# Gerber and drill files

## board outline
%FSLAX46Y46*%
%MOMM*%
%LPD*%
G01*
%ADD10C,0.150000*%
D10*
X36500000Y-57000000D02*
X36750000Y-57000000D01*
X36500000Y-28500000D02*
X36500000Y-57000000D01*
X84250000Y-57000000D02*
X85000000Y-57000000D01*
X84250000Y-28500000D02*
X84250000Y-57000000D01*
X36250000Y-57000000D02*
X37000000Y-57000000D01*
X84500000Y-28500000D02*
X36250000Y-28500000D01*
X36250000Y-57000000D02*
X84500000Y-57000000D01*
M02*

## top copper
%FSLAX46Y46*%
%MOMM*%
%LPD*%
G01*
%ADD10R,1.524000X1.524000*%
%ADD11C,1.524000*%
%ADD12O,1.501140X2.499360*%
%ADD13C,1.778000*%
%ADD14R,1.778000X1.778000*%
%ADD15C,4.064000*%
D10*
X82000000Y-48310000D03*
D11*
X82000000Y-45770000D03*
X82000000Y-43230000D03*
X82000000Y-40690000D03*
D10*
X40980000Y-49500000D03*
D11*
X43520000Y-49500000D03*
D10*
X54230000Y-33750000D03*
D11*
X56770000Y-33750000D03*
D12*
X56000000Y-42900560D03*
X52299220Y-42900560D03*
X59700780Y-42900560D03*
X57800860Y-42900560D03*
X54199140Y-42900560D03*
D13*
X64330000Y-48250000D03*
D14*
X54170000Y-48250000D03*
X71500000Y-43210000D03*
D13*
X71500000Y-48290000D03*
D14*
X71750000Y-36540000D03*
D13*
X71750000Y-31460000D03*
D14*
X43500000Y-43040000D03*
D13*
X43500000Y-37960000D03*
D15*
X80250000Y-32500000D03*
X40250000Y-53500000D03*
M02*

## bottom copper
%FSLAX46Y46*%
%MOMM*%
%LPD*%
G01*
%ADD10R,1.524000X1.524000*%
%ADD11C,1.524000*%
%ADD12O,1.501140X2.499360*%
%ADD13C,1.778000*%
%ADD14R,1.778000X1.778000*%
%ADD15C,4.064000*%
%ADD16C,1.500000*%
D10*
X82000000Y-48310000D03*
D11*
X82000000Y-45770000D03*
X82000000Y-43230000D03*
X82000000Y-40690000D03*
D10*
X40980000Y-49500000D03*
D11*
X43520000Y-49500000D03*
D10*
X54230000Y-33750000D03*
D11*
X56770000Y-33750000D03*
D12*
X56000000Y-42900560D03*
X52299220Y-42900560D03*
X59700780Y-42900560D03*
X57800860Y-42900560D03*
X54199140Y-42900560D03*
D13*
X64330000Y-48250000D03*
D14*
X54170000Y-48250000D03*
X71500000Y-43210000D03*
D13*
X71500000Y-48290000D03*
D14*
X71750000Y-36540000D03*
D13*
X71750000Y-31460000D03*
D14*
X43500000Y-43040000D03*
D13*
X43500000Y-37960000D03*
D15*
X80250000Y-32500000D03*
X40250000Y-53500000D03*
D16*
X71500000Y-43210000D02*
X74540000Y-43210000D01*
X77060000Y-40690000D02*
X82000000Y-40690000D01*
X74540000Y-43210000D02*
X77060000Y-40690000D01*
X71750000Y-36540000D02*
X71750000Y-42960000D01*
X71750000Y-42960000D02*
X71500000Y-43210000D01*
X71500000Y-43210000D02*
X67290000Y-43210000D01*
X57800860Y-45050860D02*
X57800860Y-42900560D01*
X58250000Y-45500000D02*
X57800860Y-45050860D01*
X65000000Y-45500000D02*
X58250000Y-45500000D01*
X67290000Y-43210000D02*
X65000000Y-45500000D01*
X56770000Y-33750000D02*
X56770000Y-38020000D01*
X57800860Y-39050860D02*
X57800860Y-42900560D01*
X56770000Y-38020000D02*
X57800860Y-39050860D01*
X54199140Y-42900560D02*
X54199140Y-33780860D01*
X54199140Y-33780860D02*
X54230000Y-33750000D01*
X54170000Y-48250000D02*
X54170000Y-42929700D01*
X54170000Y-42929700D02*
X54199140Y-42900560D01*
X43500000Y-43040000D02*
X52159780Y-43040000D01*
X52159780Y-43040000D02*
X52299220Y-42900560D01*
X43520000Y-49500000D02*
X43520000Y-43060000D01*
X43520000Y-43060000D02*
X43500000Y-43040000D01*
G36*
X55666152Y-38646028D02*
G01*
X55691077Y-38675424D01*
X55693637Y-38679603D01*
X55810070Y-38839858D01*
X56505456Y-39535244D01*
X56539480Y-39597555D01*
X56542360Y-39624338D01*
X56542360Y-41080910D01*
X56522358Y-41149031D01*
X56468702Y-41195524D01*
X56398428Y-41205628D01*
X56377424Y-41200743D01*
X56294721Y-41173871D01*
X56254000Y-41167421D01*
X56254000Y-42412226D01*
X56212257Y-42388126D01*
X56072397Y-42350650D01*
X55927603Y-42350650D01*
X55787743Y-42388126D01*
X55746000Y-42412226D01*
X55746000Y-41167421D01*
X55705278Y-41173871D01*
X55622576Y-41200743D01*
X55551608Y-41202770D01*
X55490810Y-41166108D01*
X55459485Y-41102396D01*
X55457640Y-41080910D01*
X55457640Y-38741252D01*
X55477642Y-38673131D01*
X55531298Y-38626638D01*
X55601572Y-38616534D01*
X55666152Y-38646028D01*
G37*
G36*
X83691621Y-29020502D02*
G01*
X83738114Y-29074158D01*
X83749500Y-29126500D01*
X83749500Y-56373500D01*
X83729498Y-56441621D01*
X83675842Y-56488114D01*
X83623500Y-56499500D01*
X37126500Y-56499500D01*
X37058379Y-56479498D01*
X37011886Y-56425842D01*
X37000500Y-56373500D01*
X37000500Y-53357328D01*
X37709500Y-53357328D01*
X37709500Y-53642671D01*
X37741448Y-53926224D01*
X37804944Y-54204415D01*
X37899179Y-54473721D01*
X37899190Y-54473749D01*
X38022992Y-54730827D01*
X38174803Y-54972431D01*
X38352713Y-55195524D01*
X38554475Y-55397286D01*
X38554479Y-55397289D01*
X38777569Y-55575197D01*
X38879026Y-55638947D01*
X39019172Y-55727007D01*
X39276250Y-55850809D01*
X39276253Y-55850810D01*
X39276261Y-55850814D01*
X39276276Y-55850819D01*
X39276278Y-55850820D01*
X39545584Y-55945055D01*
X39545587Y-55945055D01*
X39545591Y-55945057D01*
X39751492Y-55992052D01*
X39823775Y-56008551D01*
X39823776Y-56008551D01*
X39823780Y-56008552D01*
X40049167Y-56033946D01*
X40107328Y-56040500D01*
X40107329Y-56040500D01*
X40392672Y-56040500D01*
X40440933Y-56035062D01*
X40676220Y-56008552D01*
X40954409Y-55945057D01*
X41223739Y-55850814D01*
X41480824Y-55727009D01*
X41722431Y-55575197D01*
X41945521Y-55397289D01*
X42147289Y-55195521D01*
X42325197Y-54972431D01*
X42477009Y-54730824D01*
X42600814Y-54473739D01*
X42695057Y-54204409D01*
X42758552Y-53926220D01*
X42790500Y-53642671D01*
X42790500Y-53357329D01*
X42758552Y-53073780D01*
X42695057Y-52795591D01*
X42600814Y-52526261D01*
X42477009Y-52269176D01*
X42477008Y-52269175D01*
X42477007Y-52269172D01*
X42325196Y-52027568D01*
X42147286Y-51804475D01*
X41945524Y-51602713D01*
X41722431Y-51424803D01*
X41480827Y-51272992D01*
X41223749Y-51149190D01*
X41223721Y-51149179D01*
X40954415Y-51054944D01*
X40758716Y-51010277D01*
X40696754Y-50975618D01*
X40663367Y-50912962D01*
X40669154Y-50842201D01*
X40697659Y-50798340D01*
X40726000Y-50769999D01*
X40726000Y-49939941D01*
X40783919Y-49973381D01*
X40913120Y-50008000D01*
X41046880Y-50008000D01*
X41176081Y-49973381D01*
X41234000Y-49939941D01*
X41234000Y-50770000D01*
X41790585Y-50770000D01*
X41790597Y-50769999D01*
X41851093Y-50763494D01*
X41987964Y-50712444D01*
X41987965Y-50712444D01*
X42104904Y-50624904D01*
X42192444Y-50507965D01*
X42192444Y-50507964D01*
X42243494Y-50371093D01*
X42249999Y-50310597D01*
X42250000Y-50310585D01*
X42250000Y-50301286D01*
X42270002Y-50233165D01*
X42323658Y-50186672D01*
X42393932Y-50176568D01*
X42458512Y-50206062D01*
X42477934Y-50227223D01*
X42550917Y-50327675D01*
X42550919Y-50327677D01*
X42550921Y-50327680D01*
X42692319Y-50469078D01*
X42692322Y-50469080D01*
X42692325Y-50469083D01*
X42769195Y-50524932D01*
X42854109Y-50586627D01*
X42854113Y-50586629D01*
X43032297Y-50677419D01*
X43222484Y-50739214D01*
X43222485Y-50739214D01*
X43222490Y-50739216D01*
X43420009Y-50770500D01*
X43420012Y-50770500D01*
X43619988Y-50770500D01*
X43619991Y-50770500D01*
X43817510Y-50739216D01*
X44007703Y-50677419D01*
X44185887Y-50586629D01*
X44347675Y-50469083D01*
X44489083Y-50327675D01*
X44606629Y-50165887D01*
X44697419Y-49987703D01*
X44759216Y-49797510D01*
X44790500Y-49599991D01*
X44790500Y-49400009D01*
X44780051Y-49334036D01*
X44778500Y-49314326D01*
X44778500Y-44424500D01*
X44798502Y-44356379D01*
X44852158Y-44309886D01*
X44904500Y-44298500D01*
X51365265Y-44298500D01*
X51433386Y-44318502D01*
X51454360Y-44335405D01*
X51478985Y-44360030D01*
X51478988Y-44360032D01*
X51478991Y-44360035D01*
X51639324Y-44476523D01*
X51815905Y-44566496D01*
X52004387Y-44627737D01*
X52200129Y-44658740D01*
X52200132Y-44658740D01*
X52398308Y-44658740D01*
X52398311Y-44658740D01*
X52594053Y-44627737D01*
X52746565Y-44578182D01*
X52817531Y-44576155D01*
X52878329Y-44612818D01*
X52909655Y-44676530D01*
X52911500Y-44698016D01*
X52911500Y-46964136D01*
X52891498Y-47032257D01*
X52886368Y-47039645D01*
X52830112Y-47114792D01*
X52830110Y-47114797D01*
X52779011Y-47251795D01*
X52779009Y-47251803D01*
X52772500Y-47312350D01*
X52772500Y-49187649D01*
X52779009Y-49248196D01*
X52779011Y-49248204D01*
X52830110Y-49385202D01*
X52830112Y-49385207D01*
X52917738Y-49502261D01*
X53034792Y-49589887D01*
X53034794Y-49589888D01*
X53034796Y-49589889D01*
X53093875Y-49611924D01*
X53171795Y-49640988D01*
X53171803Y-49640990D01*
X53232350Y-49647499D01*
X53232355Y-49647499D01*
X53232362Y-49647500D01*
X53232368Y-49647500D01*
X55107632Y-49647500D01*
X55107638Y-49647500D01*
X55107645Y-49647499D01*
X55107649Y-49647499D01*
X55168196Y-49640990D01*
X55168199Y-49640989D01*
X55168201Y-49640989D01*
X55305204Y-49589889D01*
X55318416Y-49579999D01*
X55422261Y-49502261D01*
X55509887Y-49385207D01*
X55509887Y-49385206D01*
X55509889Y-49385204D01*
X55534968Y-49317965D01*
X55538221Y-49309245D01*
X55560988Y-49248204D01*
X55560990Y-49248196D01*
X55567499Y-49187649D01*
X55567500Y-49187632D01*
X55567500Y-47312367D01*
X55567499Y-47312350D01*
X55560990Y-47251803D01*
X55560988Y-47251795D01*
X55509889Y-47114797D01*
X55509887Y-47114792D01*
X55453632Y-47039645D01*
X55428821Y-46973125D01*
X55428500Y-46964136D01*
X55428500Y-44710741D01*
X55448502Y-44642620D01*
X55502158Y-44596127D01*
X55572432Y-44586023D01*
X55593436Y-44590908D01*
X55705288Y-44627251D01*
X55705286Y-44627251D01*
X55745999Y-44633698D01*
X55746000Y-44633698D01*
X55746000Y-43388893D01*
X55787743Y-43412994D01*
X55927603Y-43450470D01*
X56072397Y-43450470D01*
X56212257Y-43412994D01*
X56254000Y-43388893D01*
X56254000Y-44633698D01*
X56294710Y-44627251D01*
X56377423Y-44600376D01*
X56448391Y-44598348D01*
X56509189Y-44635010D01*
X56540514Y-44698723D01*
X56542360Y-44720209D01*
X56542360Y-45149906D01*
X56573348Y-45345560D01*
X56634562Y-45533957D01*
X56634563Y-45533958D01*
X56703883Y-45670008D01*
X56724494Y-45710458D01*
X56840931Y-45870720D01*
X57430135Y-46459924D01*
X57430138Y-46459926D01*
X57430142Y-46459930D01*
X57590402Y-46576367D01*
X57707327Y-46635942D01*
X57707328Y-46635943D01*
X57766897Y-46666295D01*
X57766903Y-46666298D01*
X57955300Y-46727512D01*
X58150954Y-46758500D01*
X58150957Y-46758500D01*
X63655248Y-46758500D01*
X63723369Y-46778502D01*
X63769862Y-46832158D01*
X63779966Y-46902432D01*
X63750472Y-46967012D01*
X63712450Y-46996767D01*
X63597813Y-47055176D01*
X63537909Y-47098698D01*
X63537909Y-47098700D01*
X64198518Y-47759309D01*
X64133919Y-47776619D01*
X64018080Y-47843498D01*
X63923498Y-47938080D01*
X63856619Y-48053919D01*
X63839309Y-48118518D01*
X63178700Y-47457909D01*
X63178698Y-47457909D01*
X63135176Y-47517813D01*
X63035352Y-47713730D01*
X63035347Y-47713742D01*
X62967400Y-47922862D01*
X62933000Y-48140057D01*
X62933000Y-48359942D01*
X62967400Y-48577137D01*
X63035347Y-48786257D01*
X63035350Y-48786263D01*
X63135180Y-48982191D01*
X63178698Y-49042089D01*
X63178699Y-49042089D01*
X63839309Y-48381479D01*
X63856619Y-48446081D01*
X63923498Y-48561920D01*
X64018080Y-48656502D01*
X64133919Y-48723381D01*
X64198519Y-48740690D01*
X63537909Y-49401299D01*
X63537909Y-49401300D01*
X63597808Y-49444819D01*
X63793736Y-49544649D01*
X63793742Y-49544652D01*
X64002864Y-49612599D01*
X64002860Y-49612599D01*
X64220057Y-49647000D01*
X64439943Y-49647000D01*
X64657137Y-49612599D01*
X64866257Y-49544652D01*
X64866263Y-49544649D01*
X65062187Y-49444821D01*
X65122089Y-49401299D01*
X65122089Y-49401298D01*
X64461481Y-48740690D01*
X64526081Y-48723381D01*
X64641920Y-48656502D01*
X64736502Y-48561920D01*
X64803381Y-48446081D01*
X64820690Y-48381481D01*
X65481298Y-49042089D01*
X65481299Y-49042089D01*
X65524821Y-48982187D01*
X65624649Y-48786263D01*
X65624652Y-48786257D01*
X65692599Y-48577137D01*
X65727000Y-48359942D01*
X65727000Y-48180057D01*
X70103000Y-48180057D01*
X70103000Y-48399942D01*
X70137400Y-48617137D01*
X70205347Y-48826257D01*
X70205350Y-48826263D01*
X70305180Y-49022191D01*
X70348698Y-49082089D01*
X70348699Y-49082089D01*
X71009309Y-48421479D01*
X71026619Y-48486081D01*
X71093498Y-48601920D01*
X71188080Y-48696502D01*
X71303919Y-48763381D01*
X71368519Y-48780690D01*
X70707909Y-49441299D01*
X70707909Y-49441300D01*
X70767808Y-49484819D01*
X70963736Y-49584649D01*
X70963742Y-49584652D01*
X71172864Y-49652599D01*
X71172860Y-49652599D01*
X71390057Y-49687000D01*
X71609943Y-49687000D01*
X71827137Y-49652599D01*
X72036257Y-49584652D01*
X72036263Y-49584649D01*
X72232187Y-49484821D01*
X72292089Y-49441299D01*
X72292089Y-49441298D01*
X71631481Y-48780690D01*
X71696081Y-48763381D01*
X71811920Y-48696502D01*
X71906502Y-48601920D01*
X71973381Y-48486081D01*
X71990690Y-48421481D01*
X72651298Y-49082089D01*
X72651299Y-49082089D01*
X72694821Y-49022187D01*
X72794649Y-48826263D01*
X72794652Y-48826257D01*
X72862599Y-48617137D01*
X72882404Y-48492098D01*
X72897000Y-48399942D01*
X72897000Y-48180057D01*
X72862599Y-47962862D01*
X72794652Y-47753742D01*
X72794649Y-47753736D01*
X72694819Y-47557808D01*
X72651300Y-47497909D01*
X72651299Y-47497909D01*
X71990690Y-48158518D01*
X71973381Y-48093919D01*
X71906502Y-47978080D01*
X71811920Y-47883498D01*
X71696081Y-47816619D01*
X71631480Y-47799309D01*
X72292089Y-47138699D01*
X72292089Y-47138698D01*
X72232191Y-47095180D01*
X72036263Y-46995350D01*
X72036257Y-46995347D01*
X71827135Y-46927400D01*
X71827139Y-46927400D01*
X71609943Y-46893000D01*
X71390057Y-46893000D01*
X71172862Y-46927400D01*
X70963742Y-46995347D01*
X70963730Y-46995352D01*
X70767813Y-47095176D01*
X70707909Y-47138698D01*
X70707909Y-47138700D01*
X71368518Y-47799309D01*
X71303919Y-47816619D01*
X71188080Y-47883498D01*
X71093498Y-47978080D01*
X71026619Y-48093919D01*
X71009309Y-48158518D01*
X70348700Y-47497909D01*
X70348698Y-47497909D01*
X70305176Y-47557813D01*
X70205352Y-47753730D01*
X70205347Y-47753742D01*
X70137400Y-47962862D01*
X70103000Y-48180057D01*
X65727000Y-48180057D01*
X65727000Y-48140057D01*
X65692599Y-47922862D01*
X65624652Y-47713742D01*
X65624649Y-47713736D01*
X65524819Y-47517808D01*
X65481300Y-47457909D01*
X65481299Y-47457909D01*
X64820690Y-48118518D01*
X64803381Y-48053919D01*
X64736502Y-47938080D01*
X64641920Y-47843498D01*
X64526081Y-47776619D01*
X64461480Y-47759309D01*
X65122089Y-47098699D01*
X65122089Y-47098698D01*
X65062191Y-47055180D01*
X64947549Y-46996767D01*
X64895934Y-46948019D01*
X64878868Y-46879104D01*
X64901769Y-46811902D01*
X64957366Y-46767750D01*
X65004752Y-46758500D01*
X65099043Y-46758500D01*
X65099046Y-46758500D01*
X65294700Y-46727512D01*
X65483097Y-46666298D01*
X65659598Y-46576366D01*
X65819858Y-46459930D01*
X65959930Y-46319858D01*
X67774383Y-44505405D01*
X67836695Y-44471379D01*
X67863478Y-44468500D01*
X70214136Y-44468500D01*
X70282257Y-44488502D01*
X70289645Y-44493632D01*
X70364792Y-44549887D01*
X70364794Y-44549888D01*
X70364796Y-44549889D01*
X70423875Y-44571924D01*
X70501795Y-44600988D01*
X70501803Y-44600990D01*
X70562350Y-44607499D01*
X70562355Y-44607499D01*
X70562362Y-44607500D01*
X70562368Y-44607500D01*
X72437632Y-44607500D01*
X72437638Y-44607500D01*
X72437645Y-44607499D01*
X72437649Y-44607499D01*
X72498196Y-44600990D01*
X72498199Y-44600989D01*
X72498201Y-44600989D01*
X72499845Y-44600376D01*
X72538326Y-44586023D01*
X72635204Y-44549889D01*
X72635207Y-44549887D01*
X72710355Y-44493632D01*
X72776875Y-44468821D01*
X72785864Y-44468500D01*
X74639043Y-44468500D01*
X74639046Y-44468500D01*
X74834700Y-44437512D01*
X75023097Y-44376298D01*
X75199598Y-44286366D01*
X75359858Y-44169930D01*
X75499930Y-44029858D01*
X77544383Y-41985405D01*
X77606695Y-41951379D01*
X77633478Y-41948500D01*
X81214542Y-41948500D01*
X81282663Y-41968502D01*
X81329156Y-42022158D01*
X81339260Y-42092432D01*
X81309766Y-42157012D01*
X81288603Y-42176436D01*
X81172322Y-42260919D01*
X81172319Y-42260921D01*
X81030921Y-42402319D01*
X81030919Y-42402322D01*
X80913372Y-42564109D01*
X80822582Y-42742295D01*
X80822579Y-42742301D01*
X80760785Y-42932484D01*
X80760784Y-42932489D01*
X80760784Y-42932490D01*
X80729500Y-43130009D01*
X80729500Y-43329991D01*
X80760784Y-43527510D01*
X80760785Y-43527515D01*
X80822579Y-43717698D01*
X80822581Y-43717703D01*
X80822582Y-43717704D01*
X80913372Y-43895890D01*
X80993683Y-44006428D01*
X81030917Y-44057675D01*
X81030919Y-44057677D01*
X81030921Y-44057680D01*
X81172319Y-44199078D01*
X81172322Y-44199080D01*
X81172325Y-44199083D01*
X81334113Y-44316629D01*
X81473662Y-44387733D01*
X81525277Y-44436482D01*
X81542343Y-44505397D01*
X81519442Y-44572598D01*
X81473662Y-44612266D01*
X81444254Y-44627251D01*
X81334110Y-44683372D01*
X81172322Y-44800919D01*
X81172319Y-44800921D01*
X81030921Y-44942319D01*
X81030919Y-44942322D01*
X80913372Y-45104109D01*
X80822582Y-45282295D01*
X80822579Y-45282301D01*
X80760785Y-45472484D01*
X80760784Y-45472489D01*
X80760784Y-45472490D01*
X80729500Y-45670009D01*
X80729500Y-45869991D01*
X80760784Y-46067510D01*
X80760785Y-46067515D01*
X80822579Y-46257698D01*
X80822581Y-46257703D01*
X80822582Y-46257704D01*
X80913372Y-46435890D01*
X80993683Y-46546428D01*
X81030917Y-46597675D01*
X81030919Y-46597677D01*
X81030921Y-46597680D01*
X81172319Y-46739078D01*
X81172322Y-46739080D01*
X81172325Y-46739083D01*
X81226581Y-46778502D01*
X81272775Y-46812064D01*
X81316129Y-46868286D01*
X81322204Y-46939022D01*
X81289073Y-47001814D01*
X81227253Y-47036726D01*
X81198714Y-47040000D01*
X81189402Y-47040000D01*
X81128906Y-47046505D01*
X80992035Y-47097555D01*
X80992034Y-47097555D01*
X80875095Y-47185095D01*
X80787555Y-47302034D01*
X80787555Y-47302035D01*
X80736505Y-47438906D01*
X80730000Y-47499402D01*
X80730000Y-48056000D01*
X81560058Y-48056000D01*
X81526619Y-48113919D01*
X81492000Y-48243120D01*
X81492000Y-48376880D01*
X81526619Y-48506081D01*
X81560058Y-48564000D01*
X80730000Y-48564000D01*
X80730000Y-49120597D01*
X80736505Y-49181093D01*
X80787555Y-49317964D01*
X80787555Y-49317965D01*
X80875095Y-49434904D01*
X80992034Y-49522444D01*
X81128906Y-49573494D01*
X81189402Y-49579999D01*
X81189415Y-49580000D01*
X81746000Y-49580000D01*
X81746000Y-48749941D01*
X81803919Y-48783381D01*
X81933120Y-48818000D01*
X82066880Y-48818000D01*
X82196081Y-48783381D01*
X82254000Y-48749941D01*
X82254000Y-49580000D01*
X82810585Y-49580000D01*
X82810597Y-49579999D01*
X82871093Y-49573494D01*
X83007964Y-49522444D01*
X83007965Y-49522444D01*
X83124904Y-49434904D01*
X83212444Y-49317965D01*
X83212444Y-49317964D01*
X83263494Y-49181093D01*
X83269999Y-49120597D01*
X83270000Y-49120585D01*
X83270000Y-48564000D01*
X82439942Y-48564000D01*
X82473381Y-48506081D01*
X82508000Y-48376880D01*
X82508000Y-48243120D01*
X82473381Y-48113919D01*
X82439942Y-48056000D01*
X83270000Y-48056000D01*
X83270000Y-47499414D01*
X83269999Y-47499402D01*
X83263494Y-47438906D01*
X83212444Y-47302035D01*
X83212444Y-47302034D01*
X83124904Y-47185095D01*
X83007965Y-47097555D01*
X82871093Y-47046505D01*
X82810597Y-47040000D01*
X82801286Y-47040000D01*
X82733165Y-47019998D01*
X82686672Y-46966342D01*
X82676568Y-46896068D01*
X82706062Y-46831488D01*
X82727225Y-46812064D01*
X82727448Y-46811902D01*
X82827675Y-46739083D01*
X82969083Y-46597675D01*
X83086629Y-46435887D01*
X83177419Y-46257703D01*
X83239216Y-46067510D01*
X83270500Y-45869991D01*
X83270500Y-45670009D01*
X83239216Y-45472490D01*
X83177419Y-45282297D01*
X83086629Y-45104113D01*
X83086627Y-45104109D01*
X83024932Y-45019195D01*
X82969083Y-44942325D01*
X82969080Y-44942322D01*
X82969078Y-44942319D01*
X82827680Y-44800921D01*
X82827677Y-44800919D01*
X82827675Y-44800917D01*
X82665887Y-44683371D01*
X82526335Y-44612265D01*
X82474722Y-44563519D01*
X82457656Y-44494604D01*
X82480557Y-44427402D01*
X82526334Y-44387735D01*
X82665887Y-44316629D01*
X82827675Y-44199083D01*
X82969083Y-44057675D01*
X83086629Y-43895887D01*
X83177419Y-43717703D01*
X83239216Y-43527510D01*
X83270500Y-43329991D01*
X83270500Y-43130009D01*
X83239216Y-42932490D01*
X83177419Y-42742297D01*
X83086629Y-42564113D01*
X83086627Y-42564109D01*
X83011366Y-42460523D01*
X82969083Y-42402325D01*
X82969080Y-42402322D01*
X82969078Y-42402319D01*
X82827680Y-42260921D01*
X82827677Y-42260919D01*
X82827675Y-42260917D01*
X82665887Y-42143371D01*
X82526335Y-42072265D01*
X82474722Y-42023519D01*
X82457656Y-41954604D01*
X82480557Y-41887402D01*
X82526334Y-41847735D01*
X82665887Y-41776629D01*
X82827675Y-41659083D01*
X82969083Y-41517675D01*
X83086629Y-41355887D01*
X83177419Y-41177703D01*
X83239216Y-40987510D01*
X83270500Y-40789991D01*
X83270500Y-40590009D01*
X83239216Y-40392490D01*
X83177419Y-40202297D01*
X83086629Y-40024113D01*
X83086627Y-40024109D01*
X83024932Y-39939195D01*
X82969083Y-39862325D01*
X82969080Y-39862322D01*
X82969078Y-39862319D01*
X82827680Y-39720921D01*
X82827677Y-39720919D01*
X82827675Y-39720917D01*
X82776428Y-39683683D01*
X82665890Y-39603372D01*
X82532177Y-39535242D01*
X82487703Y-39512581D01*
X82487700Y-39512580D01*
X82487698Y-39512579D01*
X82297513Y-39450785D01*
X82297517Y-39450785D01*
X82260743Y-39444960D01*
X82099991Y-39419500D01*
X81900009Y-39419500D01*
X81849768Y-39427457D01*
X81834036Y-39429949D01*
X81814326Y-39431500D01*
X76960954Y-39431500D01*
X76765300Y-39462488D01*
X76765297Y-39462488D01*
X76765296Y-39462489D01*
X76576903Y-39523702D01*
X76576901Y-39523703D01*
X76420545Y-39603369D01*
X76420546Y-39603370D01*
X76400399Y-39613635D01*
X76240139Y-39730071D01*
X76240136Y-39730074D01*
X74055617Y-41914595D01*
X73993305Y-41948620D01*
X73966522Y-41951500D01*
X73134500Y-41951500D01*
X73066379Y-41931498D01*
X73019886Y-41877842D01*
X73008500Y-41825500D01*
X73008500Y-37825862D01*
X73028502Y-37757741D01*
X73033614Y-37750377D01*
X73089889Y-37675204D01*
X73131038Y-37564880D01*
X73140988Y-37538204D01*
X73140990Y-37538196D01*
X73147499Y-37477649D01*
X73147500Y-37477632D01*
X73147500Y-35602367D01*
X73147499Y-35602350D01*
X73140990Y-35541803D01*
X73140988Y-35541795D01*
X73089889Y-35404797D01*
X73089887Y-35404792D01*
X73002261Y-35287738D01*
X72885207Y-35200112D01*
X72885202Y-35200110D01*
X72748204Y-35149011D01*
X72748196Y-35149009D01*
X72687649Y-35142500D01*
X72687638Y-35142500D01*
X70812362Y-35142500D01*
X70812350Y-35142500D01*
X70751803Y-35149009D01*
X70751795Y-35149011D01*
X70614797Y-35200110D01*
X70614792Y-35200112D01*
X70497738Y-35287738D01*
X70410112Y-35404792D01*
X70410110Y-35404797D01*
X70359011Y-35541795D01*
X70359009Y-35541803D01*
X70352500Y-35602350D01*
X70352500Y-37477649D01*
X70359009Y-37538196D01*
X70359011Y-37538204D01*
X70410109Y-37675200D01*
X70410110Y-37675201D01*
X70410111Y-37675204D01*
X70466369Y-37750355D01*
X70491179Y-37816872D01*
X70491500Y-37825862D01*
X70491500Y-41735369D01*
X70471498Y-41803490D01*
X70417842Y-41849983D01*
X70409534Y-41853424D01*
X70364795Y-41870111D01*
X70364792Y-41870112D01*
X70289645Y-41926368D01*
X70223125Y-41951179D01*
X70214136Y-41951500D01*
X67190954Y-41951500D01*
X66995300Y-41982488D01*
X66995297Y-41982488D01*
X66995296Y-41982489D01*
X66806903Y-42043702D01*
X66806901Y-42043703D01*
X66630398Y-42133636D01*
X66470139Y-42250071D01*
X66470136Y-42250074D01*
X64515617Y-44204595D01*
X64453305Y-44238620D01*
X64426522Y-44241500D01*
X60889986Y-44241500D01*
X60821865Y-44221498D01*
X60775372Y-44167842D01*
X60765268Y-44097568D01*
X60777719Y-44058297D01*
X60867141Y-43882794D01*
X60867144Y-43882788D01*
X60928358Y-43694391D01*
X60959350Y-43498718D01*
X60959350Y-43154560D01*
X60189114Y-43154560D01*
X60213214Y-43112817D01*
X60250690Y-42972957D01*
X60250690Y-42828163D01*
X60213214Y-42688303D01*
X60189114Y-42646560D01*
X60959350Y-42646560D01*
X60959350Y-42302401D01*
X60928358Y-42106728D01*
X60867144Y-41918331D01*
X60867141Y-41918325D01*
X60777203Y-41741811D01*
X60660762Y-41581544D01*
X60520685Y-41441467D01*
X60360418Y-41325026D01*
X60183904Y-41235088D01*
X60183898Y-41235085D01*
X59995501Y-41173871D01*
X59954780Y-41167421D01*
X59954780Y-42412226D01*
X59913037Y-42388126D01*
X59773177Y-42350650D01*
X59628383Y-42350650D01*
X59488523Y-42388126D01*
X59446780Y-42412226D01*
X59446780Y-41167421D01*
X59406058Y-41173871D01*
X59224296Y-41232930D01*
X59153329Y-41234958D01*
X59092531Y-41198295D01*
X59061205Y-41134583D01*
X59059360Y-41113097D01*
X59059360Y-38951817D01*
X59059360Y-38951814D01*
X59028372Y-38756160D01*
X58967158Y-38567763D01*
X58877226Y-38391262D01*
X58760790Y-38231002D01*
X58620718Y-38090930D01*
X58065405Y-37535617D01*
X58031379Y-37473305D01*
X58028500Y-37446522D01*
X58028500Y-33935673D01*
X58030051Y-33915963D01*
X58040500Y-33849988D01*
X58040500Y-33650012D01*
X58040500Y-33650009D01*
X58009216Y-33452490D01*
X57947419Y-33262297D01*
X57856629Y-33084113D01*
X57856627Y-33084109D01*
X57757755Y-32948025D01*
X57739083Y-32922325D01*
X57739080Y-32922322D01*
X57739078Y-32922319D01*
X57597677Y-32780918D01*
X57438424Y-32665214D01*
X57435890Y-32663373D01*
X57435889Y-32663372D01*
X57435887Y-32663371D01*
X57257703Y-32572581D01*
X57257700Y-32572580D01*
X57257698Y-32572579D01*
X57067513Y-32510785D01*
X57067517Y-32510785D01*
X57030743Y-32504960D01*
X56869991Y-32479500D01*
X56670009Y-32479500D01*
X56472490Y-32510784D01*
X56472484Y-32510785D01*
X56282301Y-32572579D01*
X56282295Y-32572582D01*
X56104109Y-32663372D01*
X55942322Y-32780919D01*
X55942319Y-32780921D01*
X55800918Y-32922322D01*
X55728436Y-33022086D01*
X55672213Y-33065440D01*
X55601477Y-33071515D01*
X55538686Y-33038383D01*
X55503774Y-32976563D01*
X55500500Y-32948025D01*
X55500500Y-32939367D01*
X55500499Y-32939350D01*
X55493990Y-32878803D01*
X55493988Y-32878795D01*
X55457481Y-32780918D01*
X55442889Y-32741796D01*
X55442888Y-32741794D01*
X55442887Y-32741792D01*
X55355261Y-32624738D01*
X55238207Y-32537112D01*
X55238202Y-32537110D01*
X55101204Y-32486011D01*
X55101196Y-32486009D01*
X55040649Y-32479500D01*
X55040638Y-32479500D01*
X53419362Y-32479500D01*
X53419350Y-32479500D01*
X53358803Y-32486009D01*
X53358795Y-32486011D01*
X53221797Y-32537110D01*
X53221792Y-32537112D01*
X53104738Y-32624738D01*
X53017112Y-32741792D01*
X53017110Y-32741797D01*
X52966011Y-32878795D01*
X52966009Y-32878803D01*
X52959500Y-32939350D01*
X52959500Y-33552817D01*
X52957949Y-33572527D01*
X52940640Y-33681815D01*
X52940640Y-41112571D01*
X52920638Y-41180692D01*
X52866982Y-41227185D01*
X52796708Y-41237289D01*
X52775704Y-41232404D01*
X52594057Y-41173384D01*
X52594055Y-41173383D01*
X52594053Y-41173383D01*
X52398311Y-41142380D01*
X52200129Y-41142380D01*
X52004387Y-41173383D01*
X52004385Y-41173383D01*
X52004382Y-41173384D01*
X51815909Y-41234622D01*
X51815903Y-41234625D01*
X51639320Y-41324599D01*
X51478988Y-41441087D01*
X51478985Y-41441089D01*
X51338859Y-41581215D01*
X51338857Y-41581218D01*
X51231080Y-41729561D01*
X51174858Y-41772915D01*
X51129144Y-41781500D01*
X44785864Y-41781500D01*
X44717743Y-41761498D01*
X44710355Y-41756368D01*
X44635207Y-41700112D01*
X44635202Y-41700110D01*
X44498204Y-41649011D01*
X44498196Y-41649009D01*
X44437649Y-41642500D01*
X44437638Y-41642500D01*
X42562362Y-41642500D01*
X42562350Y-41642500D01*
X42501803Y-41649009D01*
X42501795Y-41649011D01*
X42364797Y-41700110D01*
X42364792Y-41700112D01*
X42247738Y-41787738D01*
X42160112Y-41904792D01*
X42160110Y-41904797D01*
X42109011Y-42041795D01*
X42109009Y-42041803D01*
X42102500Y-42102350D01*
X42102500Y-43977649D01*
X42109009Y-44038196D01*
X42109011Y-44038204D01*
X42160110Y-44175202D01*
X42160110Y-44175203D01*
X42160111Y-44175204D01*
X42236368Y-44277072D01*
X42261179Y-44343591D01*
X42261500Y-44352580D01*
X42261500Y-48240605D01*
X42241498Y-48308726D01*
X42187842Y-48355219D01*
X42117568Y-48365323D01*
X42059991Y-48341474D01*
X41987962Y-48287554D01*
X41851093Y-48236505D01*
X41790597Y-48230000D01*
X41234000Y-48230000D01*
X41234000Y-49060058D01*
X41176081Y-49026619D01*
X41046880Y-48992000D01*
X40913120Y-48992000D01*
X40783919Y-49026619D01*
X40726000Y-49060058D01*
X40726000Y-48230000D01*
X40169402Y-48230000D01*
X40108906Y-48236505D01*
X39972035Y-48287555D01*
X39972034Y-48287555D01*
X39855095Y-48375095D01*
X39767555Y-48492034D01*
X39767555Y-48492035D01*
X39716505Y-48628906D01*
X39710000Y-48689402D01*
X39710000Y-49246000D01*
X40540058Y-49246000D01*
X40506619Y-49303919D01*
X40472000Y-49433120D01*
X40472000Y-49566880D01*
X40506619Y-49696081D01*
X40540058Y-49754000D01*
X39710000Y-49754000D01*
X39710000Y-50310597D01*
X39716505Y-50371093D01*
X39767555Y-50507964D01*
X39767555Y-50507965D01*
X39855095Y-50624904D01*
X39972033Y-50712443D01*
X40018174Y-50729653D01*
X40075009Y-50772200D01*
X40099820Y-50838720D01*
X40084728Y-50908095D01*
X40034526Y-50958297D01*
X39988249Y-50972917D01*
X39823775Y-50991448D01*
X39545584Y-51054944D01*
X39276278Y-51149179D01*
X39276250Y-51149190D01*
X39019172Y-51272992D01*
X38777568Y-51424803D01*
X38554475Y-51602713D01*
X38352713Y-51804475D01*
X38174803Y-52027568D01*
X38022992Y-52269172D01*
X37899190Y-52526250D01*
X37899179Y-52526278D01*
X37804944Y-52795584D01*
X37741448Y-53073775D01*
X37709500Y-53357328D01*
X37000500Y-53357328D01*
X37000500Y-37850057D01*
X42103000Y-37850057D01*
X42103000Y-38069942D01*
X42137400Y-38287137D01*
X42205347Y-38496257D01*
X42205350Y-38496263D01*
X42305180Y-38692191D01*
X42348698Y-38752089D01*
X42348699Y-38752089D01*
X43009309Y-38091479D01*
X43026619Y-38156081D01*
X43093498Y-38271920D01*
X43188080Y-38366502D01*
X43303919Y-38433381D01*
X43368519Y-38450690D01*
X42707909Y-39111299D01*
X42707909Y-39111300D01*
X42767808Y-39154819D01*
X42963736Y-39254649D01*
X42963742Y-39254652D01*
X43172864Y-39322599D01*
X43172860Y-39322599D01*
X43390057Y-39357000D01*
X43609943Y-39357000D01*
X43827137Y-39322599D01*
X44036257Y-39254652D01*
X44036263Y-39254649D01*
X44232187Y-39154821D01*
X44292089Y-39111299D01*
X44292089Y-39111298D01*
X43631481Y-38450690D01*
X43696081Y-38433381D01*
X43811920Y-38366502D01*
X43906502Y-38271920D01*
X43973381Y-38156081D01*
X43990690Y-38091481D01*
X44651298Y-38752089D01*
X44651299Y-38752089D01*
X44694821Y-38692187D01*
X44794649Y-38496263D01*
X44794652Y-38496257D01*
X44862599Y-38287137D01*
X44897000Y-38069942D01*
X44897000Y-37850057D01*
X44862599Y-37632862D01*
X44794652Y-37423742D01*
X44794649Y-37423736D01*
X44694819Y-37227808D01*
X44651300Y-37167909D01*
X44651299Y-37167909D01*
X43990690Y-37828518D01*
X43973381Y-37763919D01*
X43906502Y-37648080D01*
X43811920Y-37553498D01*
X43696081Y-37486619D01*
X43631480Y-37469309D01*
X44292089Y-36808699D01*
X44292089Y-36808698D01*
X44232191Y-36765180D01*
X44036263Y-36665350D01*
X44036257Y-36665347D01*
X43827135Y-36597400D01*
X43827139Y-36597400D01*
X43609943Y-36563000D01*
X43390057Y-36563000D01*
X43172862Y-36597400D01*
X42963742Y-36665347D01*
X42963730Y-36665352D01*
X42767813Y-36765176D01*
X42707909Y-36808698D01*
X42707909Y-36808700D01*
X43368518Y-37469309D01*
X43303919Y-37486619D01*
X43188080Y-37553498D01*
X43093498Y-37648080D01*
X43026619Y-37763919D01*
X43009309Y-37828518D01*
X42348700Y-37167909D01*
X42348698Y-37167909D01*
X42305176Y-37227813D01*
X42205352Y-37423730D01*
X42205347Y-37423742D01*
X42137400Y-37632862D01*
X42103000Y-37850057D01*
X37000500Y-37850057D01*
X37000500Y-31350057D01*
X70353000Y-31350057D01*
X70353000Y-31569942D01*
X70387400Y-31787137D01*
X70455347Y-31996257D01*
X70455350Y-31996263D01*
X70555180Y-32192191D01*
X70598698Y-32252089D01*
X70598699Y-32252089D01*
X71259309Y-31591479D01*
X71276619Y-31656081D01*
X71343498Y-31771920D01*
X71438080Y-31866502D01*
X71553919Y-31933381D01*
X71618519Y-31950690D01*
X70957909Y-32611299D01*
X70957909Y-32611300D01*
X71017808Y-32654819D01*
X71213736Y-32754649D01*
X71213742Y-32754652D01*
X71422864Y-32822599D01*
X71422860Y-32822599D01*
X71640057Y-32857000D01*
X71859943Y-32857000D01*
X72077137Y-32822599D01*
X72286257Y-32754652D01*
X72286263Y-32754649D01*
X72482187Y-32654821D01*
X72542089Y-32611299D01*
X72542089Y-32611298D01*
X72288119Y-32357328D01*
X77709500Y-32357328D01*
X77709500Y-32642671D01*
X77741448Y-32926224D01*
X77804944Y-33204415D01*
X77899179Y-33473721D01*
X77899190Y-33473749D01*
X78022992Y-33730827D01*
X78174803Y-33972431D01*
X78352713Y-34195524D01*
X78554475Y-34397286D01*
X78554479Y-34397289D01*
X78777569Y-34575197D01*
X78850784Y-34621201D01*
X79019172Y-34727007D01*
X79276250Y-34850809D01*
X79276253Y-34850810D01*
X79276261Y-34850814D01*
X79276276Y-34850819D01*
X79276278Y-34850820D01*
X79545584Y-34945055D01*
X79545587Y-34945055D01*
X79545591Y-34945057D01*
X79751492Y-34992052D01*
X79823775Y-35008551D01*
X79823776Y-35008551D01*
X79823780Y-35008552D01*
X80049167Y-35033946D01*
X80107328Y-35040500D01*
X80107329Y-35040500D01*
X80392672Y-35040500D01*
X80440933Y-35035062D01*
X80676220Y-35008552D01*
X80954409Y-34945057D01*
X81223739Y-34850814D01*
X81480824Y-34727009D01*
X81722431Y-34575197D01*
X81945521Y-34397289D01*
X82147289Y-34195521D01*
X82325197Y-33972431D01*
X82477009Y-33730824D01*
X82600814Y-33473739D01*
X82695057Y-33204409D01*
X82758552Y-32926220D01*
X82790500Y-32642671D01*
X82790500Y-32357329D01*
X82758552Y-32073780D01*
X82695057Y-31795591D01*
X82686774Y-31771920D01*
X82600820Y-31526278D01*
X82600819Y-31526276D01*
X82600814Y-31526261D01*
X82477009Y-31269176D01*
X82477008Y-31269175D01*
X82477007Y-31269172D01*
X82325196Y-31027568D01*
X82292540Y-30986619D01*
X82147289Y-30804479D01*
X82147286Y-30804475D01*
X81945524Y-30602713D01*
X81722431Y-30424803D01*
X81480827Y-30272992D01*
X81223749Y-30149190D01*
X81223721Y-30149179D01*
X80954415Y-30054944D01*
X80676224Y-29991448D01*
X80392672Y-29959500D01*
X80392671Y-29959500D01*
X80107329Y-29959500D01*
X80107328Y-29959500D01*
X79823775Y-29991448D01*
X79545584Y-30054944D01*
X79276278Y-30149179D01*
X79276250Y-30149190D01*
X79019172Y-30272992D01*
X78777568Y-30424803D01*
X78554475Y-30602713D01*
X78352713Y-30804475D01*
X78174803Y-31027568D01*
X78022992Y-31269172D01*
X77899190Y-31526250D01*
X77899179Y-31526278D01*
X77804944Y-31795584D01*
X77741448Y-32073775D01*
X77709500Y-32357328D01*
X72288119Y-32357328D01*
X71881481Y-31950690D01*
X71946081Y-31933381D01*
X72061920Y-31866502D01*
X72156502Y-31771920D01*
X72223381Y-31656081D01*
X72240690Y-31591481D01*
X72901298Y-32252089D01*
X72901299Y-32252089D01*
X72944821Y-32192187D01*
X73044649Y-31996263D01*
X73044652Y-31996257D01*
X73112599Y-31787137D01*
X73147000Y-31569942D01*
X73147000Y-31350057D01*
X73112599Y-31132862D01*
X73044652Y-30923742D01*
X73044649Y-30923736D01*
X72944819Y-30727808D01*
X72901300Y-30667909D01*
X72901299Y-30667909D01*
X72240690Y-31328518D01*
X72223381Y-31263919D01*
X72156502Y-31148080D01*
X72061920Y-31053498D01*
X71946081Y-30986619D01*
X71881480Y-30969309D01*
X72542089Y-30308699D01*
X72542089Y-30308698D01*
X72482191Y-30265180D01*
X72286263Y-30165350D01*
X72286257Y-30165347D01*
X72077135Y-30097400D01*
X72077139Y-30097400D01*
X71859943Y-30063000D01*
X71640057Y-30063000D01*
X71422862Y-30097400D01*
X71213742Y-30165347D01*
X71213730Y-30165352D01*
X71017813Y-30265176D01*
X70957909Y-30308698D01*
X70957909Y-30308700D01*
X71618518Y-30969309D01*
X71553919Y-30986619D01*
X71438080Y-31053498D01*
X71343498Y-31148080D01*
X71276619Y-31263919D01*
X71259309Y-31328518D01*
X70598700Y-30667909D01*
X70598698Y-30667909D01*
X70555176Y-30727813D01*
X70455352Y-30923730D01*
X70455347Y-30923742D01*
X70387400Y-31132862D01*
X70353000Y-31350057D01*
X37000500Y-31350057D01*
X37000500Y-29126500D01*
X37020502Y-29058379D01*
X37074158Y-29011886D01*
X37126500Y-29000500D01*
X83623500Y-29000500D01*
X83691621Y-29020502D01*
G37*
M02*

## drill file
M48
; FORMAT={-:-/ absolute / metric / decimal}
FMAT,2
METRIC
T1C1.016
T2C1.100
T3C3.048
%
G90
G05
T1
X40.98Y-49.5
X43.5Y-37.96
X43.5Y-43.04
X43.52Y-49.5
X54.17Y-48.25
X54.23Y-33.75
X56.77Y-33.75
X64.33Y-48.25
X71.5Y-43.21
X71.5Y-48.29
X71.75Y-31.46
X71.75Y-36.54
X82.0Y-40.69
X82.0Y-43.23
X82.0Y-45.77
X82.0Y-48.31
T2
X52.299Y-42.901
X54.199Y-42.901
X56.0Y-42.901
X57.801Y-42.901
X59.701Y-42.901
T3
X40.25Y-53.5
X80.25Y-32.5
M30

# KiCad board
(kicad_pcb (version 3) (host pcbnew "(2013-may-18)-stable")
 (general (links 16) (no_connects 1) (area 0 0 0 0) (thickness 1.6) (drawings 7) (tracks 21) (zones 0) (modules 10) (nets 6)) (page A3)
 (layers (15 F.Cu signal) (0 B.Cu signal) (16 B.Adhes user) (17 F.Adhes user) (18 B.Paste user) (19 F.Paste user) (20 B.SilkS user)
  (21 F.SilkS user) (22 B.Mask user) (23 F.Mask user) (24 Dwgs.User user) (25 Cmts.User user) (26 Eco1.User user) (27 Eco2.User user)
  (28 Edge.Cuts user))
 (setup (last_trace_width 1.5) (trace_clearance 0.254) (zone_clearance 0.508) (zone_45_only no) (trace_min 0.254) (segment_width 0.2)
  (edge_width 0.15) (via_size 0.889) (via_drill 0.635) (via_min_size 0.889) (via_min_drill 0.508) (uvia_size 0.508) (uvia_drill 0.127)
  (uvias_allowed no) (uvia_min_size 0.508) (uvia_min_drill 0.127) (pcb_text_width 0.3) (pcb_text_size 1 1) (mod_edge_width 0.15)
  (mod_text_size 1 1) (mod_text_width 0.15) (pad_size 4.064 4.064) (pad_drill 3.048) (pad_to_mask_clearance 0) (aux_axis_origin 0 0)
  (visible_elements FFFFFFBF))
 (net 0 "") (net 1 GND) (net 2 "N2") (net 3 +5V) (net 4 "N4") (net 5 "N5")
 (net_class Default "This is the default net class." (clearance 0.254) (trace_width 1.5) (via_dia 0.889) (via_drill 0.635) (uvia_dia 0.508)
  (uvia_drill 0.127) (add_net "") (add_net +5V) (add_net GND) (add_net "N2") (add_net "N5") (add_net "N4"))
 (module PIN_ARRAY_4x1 (layer F.Cu) (at 82 44.5 90)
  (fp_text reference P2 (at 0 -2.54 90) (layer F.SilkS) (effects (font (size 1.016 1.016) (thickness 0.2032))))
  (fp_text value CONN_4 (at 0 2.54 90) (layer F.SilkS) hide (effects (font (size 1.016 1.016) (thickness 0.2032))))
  (pad 1 thru_hole rect (at -3.81 0 90) (size 1.524 1.524) (drill 1.016) (layers *.Cu *.Mask F.SilkS) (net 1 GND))
  (pad 2 thru_hole circle (at -1.27 0 90) (size 1.524 1.524) (drill 1.016) (layers *.Cu *.Mask F.SilkS) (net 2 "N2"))
  (pad 3 thru_hole circle (at 1.27 0 90) (size 1.524 1.524) (drill 1.016) (layers *.Cu *.Mask F.SilkS) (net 2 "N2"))
  (pad 4 thru_hole circle (at 3.81 0 90) (size 1.524 1.524) (drill 1.016) (layers *.Cu *.Mask F.SilkS) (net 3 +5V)))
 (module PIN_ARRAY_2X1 (layer F.Cu) (at 42.25 49.5)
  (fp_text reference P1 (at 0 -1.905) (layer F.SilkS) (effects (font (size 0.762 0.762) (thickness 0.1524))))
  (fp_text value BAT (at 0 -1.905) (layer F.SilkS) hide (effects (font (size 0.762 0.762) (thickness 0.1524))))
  (pad 1 thru_hole rect (at -1.27 0) (size 1.524 1.524) (drill 1.016) (layers *.Cu *.Mask F.SilkS) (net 1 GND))
  (pad 2 thru_hole circle (at 1.27 0) (size 1.524 1.524) (drill 1.016) (layers *.Cu *.Mask F.SilkS) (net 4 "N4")))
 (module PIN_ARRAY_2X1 (layer F.Cu) (at 55.5 33.75)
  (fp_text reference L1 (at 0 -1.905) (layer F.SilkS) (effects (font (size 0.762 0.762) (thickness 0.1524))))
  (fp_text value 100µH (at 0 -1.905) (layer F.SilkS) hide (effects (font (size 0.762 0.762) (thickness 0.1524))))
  (pad 1 thru_hole rect (at -1.27 0) (size 1.524 1.524) (drill 1.016) (layers *.Cu *.Mask F.SilkS) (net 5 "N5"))
  (pad 2 thru_hole circle (at 1.27 0) (size 1.524 1.524) (drill 1.016) (layers *.Cu *.Mask F.SilkS) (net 3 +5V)))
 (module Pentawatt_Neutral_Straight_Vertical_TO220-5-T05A (layer F.Cu) (at 56 43.5)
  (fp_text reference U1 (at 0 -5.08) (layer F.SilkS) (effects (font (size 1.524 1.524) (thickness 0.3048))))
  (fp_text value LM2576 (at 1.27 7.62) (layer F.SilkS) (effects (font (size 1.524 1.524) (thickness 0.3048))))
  (pad 3 thru_hole oval (at 0 -0.59944 90) (size 2.49936 1.50114) (drill 1.09982) (layers *.Cu *.Mask F.SilkS) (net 1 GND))
  (pad 1 thru_hole oval (at -3.70078 -0.59944 90) (size 2.49936 1.50114) (drill 1.09982) (layers *.Cu *.Mask F.SilkS) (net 4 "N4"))
  (pad 5 thru_hole oval (at 3.70078 -0.59944 90) (size 2.49936 1.50114) (drill 1.09982) (layers *.Cu *.Mask F.SilkS) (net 1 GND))
  (pad 4 thru_hole oval (at 1.80086 -0.59944 90) (size 2.49936 1.50114) (drill 1.09982) (layers *.Cu *.Mask F.SilkS) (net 3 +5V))
  (pad 2 thru_hole oval (at -1.80086 -0.59944 90) (size 2.49936 1.50114) (drill 1.09982) (layers *.Cu *.Mask F.SilkS) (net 5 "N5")))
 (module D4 (layer F.Cu) (at 59.25 48.25 180)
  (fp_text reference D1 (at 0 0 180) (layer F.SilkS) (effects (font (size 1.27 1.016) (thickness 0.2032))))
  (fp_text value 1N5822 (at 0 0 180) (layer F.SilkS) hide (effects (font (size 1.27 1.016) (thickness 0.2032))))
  (pad 1 thru_hole circle (at -5.08 0 180) (size 1.778 1.778) (drill 1.016) (layers *.Cu *.Mask F.SilkS) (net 1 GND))
  (pad 2 thru_hole rect (at 5.08 0 180) (size 1.778 1.778) (drill 1.016) (layers *.Cu *.Mask F.SilkS) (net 5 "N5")))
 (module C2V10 (layer F.Cu) (at 71.5 45.75 270)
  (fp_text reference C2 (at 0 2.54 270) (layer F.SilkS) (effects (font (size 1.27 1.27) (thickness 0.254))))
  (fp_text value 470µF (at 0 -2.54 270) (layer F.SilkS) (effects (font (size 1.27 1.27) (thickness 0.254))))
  (pad 1 thru_hole rect (at -2.54 0 270) (size 1.778 1.778) (drill 1.016) (layers *.Cu *.Mask F.SilkS) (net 3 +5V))
  (pad 2 thru_hole circle (at 2.54 0 270) (size 1.778 1.778) (drill 1.016) (layers *.Cu *.Mask F.SilkS) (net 1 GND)))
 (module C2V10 (layer F.Cu) (at 71.75 34 90)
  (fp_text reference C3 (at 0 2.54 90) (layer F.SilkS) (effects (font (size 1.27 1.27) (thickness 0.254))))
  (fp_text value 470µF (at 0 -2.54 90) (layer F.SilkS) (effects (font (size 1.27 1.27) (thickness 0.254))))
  (pad 1 thru_hole rect (at -2.54 0 90) (size 1.778 1.778) (drill 1.016) (layers *.Cu *.Mask F.SilkS) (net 3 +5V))
  (pad 2 thru_hole circle (at 2.54 0 90) (size 1.778 1.778) (drill 1.016) (layers *.Cu *.Mask F.SilkS) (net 1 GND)))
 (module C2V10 (layer F.Cu) (at 43.5 40.5 90)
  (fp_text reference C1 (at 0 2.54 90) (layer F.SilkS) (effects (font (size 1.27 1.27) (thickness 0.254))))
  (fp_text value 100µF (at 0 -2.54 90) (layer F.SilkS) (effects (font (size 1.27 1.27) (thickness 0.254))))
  (pad 1 thru_hole rect (at -2.54 0 90) (size 1.778 1.778) (drill 1.016) (layers *.Cu *.Mask F.SilkS) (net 4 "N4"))
  (pad 2 thru_hole circle (at 2.54 0 90) (size 1.778 1.778) (drill 1.016) (layers *.Cu *.Mask F.SilkS) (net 1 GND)))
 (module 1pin (layer F.Cu) (at 80.25 32.5)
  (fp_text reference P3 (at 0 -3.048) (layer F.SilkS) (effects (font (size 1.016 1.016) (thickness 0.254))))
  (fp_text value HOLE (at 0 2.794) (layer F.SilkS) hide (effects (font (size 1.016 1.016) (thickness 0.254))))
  (pad 1 thru_hole circle (at 0 0) (size 4.064 4.064) (drill 3.048) (layers *.Cu *.Mask F.SilkS)))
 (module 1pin (layer F.Cu) (at 40.25 53.5)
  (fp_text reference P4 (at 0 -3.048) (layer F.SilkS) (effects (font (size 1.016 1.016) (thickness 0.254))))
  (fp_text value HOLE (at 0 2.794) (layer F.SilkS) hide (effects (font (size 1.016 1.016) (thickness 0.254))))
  (pad 1 thru_hole circle (at 0 0) (size 4.064 4.064) (drill 3.048) (layers *.Cu *.Mask F.SilkS)))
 (gr_line (start 36.5 57) (end 36.75 57) (angle 90) (layer Edge.Cuts) (width 0.15))
 (gr_line (start 36.5 28.5) (end 36.5 57) (angle 90) (layer Edge.Cuts) (width 0.15))
 (gr_line (start 84.25 57) (end 85 57) (angle 90) (layer Edge.Cuts) (width 0.15))
 (gr_line (start 84.25 28.5) (end 84.25 57) (angle 90) (layer Edge.Cuts) (width 0.15))
 (gr_line (start 36.25 57) (end 37 57) (angle 90) (layer Edge.Cuts) (width 0.15))
 (gr_line (start 84.5 28.5) (end 36.25 28.5) (angle 90) (layer Edge.Cuts) (width 0.15))
 (gr_line (start 36.25 57) (end 84.5 57) (angle 90) (layer Edge.Cuts) (width 0.15))
 (segment (start 71.5 43.21) (end 74.54 43.21) (width 1.5) (layer B.Cu) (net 3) (status 10))
 (segment (start 77.06 40.69) (end 82 40.69) (width 1.5) (layer B.Cu) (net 3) (status 20))
 (segment (start 74.54 43.21) (end 77.06 40.69) (width 1.5) (layer B.Cu) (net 3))
 (segment (start 71.75 36.54) (end 71.75 42.96) (width 1.5) (layer B.Cu) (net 3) (status 30))
 (segment (start 71.75 42.96) (end 71.5 43.21) (width 1.5) (layer B.Cu) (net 3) (status 30))
 (segment (start 71.5 43.21) (end 67.29 43.21) (width 1.5) (layer B.Cu) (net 3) (status 10))
 (segment (start 57.80086 45.05086) (end 57.80086 42.90056) (width 1.5) (layer B.Cu) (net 3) (status 20))
 (segment (start 58.25 45.5) (end 57.80086 45.05086) (width 1.5) (layer B.Cu) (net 3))
 (segment (start 65 45.5) (end 58.25 45.5) (width 1.5) (layer B.Cu) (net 3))
 (segment (start 67.29 43.21) (end 65 45.5) (width 1.5) (layer B.Cu) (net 3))
 (segment (start 56.77 33.75) (end 56.77 38.02) (width 1.5) (layer B.Cu) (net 3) (status 10))
 (segment (start 57.80086 39.05086) (end 57.80086 42.90056) (width 1.5) (layer B.Cu) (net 3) (status 20))
 (segment (start 56.77 38.02) (end 57.80086 39.05086) (width 1.5) (layer B.Cu) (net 3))
 (segment (start 54.19914 42.90056) (end 54.19914 33.78086) (width 1.5) (layer B.Cu) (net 5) (status 30))
 (segment (start 54.19914 33.78086) (end 54.23 33.75) (width 1.5) (layer B.Cu) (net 5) (status 30))
 (segment (start 54.17 48.25) (end 54.17 42.9297) (width 1.5) (layer B.Cu) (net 5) (status 30))
 (segment (start 54.17 42.9297) (end 54.19914 42.90056) (width 1.5) (layer B.Cu) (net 5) (status 30))
 (segment (start 43.5 43.04) (end 52.15978 43.04) (width 1.5) (layer B.Cu) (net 4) (status 30))
 (segment (start 52.15978 43.04) (end 52.29922 42.90056) (width 1.5) (layer B.Cu) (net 4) (status 30))
 (segment (start 43.52 49.5) (end 43.52 43.06) (width 1.5) (layer B.Cu) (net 4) (status 30))
 (segment (start 43.52 43.06) (end 43.5 43.04) (width 1.5) (layer B.Cu) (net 4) (status 30))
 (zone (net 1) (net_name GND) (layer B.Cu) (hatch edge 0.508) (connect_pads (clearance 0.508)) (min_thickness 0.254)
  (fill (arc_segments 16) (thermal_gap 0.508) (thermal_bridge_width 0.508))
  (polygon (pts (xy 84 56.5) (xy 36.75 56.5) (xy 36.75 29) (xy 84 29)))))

